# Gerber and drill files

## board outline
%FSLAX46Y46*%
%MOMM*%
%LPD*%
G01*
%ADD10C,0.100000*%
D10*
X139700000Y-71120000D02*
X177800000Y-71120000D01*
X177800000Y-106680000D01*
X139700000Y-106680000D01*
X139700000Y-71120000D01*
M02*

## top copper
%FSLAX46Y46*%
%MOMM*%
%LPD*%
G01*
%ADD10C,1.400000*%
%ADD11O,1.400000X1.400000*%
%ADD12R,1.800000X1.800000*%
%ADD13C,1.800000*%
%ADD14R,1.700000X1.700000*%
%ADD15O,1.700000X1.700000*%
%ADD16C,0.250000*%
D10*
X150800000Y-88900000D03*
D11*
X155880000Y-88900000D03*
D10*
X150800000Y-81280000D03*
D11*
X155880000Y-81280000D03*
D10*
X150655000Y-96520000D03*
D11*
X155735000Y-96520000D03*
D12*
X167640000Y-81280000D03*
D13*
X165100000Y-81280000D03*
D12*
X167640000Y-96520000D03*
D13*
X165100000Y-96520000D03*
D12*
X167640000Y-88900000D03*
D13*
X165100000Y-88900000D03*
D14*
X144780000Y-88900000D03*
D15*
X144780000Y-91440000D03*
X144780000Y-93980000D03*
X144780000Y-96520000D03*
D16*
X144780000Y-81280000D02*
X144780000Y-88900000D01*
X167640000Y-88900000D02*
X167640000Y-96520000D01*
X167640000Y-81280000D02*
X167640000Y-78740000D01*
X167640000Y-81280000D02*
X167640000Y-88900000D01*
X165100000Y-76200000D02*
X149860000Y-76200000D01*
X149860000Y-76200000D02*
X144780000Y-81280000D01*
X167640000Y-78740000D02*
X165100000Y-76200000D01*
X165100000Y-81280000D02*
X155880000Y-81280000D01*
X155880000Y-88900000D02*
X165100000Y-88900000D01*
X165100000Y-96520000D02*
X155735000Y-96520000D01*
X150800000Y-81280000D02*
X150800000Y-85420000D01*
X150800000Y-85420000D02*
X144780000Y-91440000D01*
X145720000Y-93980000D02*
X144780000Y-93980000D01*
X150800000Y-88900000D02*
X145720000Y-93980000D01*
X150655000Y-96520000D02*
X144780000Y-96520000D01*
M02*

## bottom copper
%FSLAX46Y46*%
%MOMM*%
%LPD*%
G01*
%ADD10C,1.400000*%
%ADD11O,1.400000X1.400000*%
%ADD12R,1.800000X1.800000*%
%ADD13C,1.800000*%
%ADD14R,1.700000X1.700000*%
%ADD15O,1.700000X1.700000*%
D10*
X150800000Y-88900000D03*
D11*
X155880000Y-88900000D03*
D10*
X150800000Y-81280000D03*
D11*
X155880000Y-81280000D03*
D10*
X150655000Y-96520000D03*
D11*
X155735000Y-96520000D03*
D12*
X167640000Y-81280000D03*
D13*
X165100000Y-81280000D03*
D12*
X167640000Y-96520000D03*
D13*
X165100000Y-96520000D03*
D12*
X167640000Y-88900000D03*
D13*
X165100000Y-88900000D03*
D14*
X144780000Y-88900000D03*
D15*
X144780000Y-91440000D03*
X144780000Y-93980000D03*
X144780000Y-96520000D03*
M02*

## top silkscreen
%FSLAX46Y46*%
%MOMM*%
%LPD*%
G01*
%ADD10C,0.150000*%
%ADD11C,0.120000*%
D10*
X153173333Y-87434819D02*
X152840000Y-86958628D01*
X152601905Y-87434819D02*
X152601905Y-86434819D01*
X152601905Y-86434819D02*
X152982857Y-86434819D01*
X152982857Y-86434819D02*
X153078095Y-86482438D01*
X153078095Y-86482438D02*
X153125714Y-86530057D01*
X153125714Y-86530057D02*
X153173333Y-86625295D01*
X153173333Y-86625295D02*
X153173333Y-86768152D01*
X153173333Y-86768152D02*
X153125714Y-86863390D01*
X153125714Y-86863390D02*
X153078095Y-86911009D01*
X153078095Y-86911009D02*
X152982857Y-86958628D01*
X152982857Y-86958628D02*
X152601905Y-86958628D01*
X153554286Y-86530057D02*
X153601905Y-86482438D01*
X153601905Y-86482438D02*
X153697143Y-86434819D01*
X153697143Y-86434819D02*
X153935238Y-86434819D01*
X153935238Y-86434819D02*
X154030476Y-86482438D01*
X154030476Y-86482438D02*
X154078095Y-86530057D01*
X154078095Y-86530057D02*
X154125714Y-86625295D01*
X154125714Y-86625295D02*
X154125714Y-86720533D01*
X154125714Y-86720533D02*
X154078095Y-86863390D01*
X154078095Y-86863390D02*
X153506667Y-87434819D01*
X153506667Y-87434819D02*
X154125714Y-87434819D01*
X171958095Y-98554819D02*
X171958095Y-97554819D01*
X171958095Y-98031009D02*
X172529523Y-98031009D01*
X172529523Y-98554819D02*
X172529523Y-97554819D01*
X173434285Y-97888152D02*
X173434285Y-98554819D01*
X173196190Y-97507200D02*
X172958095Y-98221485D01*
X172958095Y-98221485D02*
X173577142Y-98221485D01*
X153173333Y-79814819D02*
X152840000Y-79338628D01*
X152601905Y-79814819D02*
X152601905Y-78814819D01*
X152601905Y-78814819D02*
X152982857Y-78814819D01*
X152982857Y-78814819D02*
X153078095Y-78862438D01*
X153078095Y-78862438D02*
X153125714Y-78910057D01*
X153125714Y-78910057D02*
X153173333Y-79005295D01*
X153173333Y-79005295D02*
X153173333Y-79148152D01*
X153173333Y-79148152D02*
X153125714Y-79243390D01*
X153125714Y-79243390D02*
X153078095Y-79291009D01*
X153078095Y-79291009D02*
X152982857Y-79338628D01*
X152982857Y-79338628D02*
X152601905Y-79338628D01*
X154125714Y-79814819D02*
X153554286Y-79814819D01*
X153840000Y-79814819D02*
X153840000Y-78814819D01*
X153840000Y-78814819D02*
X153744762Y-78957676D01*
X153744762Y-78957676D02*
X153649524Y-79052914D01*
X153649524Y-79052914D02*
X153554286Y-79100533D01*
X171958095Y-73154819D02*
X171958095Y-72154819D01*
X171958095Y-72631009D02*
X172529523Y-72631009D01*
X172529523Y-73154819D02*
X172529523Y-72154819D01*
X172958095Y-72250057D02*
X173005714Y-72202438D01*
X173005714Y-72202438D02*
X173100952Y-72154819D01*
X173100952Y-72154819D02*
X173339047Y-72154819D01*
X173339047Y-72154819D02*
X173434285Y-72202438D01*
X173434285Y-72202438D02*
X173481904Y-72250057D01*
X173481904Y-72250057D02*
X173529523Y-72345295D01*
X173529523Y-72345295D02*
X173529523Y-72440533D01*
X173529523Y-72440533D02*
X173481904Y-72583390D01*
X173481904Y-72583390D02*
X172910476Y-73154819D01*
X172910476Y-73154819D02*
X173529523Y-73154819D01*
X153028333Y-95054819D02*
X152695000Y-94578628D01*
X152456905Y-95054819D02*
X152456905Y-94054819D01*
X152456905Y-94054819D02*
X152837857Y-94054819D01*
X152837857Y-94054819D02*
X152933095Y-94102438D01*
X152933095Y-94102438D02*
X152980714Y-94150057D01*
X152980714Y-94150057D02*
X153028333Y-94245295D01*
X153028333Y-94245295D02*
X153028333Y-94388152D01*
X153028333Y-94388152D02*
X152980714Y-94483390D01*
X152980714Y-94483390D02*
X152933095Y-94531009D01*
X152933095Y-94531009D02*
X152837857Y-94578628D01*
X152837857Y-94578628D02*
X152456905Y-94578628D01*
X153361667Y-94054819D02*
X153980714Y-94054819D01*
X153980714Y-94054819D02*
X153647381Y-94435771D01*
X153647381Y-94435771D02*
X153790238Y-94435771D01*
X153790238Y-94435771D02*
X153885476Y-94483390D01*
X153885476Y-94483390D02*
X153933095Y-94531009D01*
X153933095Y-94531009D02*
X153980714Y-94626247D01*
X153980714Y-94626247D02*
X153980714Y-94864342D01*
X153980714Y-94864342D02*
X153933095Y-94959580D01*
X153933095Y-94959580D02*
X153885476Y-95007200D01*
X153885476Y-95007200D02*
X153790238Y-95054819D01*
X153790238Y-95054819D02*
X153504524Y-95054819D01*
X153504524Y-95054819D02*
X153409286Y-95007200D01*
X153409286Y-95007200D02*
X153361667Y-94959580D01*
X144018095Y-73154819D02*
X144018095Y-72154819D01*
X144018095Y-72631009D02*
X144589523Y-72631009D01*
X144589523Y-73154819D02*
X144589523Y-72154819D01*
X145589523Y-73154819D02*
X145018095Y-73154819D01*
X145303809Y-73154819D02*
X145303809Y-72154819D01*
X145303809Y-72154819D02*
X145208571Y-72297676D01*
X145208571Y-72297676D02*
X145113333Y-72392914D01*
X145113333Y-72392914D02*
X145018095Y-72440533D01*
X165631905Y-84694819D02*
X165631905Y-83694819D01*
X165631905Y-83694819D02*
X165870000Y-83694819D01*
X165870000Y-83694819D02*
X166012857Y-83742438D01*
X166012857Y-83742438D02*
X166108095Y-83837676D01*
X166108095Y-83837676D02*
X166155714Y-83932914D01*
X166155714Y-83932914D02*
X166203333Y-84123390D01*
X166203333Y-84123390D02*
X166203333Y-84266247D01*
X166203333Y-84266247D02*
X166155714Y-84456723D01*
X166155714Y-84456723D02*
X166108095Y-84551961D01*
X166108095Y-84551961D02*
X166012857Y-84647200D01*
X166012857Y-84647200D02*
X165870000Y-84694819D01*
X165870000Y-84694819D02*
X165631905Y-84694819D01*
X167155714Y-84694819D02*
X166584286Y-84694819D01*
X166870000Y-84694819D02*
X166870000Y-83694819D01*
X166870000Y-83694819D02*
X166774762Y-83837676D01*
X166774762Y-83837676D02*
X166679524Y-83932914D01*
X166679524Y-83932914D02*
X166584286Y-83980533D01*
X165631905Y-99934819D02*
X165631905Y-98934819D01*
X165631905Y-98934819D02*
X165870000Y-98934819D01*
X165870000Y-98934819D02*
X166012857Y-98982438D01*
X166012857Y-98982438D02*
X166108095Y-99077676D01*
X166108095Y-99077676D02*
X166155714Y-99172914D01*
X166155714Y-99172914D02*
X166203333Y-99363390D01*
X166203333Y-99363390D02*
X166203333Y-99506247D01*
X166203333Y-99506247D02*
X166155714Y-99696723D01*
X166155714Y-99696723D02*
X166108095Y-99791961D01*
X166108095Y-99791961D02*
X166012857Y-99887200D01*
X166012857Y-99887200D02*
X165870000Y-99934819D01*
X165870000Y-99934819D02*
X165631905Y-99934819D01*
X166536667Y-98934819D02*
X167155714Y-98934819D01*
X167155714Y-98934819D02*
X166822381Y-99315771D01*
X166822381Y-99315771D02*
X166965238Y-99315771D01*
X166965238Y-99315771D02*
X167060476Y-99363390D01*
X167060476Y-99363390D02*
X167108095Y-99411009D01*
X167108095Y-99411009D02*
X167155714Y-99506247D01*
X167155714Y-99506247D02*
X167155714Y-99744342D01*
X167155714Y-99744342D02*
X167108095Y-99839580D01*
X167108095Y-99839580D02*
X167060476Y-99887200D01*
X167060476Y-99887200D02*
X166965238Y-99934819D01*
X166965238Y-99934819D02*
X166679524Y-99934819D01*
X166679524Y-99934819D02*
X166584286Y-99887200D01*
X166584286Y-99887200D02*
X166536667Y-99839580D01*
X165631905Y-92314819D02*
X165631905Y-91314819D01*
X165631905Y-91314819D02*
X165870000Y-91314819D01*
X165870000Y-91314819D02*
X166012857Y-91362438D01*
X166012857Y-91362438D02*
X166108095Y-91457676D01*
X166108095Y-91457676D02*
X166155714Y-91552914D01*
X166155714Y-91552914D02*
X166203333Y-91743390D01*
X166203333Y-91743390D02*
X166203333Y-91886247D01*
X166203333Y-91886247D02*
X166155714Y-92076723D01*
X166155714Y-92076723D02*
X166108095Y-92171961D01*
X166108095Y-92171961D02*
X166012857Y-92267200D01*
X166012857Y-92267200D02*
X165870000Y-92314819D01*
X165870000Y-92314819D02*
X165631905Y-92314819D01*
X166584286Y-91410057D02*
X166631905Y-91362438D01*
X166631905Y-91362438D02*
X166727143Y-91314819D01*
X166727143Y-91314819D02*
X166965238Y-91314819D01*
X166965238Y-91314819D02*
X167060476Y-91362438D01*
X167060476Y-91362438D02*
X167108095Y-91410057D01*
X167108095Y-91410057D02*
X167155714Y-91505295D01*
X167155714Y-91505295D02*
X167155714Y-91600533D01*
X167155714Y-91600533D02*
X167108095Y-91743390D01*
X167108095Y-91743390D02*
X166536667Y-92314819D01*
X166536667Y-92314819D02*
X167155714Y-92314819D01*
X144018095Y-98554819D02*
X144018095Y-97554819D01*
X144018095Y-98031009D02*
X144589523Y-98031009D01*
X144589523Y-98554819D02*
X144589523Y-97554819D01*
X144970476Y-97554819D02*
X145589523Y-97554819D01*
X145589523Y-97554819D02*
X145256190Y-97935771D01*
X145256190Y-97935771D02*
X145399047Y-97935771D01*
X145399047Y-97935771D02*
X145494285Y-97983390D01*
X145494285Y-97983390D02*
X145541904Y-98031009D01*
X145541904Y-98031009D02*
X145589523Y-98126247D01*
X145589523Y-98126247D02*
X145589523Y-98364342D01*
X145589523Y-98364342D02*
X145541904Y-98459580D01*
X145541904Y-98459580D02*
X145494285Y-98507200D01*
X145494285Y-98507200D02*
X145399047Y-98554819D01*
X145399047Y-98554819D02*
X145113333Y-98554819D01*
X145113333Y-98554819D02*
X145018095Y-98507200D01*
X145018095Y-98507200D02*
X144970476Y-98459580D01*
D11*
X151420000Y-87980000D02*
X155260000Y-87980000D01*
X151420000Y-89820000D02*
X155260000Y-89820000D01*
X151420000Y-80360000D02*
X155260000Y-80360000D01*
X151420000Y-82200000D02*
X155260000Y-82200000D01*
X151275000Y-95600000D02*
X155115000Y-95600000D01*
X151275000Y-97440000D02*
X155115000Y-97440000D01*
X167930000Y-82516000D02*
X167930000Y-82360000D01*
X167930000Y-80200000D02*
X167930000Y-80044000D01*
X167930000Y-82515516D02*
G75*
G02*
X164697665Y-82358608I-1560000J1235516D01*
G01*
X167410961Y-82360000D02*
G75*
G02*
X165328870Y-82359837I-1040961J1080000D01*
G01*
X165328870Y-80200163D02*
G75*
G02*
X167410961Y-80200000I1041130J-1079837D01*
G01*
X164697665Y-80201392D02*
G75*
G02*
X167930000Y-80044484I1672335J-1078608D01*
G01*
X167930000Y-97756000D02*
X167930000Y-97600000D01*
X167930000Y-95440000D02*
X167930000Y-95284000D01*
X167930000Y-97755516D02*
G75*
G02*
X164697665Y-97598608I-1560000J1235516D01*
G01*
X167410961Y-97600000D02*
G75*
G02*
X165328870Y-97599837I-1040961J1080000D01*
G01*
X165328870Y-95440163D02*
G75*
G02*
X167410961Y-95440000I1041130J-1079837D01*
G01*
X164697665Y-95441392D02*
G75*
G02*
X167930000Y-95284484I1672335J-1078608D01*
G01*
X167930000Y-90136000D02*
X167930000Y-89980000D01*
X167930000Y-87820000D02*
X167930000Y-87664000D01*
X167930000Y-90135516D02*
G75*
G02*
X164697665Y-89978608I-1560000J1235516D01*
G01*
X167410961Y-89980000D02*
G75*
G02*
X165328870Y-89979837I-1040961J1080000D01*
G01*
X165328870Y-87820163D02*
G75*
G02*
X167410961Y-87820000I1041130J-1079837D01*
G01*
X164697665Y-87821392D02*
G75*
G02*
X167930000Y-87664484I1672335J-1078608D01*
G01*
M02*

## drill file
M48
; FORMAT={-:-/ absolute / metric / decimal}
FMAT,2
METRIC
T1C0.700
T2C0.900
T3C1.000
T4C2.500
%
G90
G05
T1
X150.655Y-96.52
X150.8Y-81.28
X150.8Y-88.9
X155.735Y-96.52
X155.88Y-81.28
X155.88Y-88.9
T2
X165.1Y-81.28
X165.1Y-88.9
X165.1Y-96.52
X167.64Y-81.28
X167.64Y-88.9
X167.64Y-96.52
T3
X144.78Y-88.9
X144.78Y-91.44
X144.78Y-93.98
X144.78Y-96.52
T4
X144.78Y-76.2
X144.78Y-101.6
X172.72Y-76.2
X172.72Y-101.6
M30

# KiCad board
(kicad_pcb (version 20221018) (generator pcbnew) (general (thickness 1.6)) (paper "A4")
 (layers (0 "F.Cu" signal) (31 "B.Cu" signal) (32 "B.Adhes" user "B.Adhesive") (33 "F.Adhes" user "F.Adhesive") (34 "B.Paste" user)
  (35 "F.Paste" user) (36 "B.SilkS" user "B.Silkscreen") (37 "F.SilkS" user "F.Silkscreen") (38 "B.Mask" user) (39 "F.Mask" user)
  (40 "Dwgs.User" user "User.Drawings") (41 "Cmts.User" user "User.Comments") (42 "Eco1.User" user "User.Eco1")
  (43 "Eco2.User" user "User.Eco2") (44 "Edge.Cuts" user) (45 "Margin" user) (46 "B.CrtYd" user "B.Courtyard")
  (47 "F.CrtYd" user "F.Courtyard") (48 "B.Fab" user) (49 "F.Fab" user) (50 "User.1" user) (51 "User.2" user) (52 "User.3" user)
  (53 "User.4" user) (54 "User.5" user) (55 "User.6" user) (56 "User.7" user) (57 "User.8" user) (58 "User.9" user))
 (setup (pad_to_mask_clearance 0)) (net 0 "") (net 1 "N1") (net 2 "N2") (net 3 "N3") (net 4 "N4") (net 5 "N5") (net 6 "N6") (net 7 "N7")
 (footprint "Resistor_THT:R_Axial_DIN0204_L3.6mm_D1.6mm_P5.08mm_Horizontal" (layer "F.Cu") (at 150.8 88.9)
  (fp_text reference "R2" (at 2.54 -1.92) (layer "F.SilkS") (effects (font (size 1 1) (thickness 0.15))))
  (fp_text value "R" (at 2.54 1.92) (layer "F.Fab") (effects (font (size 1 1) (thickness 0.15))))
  (fp_line (start 0.62 -0.92) (end 4.46 -0.92) (stroke (width 0.12) (type solid)) (layer "F.SilkS"))
  (fp_line (start 0.62 0.92) (end 4.46 0.92) (stroke (width 0.12) (type solid)) (layer "F.SilkS"))
  (pad "1" thru_hole circle (at 0 0) (size 1.4 1.4) (drill 0.7) (layers "*.Cu" "*.Mask") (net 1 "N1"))
  (pad "2" thru_hole oval (at 5.08 0) (size 1.4 1.4) (drill 0.7) (layers "*.Cu" "*.Mask") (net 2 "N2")))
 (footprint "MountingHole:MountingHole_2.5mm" (layer "F.Cu") (at 172.72 101.6)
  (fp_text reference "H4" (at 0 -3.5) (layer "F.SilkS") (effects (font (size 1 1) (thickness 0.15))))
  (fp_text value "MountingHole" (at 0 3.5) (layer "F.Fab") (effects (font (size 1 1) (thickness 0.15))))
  (pad "" np_thru_hole circle (at 0 0) (size 2.5 2.5) (drill 2.5) (layers "*.Cu" "*.Mask")))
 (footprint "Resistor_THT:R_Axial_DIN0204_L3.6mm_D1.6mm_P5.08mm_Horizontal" (layer "F.Cu") (at 150.8 81.28)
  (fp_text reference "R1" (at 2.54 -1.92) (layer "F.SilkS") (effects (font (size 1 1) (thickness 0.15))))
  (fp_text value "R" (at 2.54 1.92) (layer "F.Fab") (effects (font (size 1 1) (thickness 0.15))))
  (fp_line (start 0.62 -0.92) (end 4.46 -0.92) (stroke (width 0.12) (type solid)) (layer "F.SilkS"))
  (fp_line (start 0.62 0.92) (end 4.46 0.92) (stroke (width 0.12) (type solid)) (layer "F.SilkS"))
  (pad "1" thru_hole circle (at 0 0) (size 1.4 1.4) (drill 0.7) (layers "*.Cu" "*.Mask") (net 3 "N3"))
  (pad "2" thru_hole oval (at 5.08 0) (size 1.4 1.4) (drill 0.7) (layers "*.Cu" "*.Mask") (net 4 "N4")))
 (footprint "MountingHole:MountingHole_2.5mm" (layer "F.Cu") (at 172.72 76.2)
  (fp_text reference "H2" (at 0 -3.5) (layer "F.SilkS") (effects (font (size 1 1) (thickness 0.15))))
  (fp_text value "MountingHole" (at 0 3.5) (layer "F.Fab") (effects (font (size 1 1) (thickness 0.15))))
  (pad "" np_thru_hole circle (at 0 0) (size 2.5 2.5) (drill 2.5) (layers "*.Cu" "*.Mask")))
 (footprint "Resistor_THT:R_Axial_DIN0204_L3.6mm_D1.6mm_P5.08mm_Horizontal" (layer "F.Cu") (at 150.655 96.52)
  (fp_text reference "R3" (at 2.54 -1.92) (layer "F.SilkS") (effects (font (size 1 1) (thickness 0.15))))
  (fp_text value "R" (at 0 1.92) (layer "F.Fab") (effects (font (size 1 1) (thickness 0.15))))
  (fp_line (start 0.62 -0.92) (end 4.46 -0.92) (stroke (width 0.12) (type solid)) (layer "F.SilkS"))
  (fp_line (start 0.62 0.92) (end 4.46 0.92) (stroke (width 0.12) (type solid)) (layer "F.SilkS"))
  (pad "1" thru_hole circle (at 0 0) (size 1.4 1.4) (drill 0.7) (layers "*.Cu" "*.Mask") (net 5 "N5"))
  (pad "2" thru_hole oval (at 5.08 0) (size 1.4 1.4) (drill 0.7) (layers "*.Cu" "*.Mask") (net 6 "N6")))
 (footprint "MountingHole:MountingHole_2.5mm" (layer "F.Cu") (at 144.78 76.2)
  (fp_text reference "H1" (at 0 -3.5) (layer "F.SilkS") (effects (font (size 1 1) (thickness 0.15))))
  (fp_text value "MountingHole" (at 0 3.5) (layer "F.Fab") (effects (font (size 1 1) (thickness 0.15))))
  (pad "" np_thru_hole circle (at 0 0) (size 2.5 2.5) (drill 2.5) (layers "*.Cu" "*.Mask")))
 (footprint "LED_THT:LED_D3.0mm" (layer "F.Cu") (at 167.64 81.28 180)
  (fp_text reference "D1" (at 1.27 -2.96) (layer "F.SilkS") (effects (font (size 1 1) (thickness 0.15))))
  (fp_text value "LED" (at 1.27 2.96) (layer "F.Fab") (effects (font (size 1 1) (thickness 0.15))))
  (fp_line (start -0.29 -1.236) (end -0.29 -1.08) (stroke (width 0.12) (type solid)) (layer "F.SilkS"))
  (fp_line (start -0.29 1.08) (end -0.29 1.236) (stroke (width 0.12) (type solid)) (layer "F.SilkS"))
  (fp_arc (start -0.29 -1.235516) (mid 1.366487 -1.987659) (end 2.942335 -1.078608) (stroke (width 0.12) (type solid)) (layer "F.SilkS"))
  (fp_arc (start 0.229039 -1.08) (mid 1.270117 -1.5) (end 2.31113 -1.079837) (stroke (width 0.12) (type solid)) (layer "F.SilkS"))
  (fp_arc (start 2.31113 1.079837) (mid 1.270117 1.5) (end 0.229039 1.08) (stroke (width 0.12) (type solid)) (layer "F.SilkS"))
  (fp_arc (start 2.942335 1.078608) (mid 1.366487 1.987659) (end -0.29 1.235516) (stroke (width 0.12) (type solid)) (layer "F.SilkS"))
  (pad "1" thru_hole rect (at 0 0 180) (size 1.8 1.8) (drill 0.9) (layers "*.Cu" "*.Mask") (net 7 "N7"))
  (pad "2" thru_hole circle (at 2.54 0 180) (size 1.8 1.8) (drill 0.9) (layers "*.Cu" "*.Mask") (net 4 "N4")))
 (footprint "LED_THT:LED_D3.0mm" (layer "F.Cu") (at 167.64 96.52 180)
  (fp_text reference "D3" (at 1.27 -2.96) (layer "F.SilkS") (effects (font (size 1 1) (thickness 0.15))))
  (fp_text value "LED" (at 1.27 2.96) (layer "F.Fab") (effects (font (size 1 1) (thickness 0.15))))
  (fp_line (start -0.29 -1.236) (end -0.29 -1.08) (stroke (width 0.12) (type solid)) (layer "F.SilkS"))
  (fp_line (start -0.29 1.08) (end -0.29 1.236) (stroke (width 0.12) (type solid)) (layer "F.SilkS"))
  (fp_arc (start -0.29 -1.235516) (mid 1.366487 -1.987659) (end 2.942335 -1.078608) (stroke (width 0.12) (type solid)) (layer "F.SilkS"))
  (fp_arc (start 0.229039 -1.08) (mid 1.270117 -1.5) (end 2.31113 -1.079837) (stroke (width 0.12) (type solid)) (layer "F.SilkS"))
  (fp_arc (start 2.31113 1.079837) (mid 1.270117 1.5) (end 0.229039 1.08) (stroke (width 0.12) (type solid)) (layer "F.SilkS"))
  (fp_arc (start 2.942335 1.078608) (mid 1.366487 1.987659) (end -0.29 1.235516) (stroke (width 0.12) (type solid)) (layer "F.SilkS"))
  (pad "1" thru_hole rect (at 0 0 180) (size 1.8 1.8) (drill 0.9) (layers "*.Cu" "*.Mask") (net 7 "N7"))
  (pad "2" thru_hole circle (at 2.54 0 180) (size 1.8 1.8) (drill 0.9) (layers "*.Cu" "*.Mask") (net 6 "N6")))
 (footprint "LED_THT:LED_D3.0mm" (layer "F.Cu") (at 167.64 88.9 180)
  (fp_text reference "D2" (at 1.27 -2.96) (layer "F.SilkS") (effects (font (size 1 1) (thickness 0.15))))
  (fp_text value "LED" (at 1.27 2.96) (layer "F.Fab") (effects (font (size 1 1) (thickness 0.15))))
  (fp_line (start -0.29 -1.236) (end -0.29 -1.08) (stroke (width 0.12) (type solid)) (layer "F.SilkS"))
  (fp_line (start -0.29 1.08) (end -0.29 1.236) (stroke (width 0.12) (type solid)) (layer "F.SilkS"))
  (fp_arc (start -0.29 -1.235516) (mid 1.366487 -1.987659) (end 2.942335 -1.078608) (stroke (width 0.12) (type solid)) (layer "F.SilkS"))
  (fp_arc (start 0.229039 -1.08) (mid 1.270117 -1.5) (end 2.31113 -1.079837) (stroke (width 0.12) (type solid)) (layer "F.SilkS"))
  (fp_arc (start 2.31113 1.079837) (mid 1.270117 1.5) (end 0.229039 1.08) (stroke (width 0.12) (type solid)) (layer "F.SilkS"))
  (fp_arc (start 2.942335 1.078608) (mid 1.366487 1.987659) (end -0.29 1.235516) (stroke (width 0.12) (type solid)) (layer "F.SilkS"))
  (pad "1" thru_hole rect (at 0 0 180) (size 1.8 1.8) (drill 0.9) (layers "*.Cu" "*.Mask") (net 7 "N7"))
  (pad "2" thru_hole circle (at 2.54 0 180) (size 1.8 1.8) (drill 0.9) (layers "*.Cu" "*.Mask") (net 2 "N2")))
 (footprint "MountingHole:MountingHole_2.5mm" (layer "F.Cu") (at 144.78 101.6)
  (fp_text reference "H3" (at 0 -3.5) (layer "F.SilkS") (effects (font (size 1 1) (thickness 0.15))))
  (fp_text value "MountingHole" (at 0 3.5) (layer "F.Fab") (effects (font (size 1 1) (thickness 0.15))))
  (pad "" np_thru_hole circle (at 0 0) (size 2.5 2.5) (drill 2.5) (layers "*.Cu" "*.Mask")))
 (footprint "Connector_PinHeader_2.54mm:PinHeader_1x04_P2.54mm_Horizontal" (layer "B.Cu") (at 144.78 88.9 180)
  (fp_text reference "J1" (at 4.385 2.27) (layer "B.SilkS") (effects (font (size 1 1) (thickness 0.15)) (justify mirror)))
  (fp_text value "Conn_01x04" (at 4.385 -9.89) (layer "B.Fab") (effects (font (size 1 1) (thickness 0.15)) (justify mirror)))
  (pad "1" thru_hole rect (at 0 0 180) (size 1.7 1.7) (drill 1) (layers "*.Cu" "*.Mask") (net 7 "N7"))
  (pad "2" thru_hole oval (at 0 -2.54 180) (size 1.7 1.7) (drill 1) (layers "*.Cu" "*.Mask") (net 3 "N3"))
  (pad "3" thru_hole oval (at 0 -5.08 180) (size 1.7 1.7) (drill 1) (layers "*.Cu" "*.Mask") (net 1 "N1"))
  (pad "4" thru_hole oval (at 0 -7.62 180) (size 1.7 1.7) (drill 1) (layers "*.Cu" "*.Mask") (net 5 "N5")))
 (gr_poly
  (pts (xy 139.7 71.12) (xy 177.8 71.12) (xy 177.8 106.68) (xy 139.7 106.68)) (stroke (width 0.1) (type solid)) (fill none)
  (layer "Edge.Cuts"))
 (segment (start 144.78 81.28) (end 144.78 88.9) (width 0.25) (layer "F.Cu") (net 7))
 (segment (start 167.64 88.9) (end 167.64 96.52) (width 0.25) (layer "F.Cu") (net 7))
 (segment (start 167.64 81.28) (end 167.64 78.74) (width 0.25) (layer "F.Cu") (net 7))
 (segment (start 167.64 81.28) (end 167.64 88.9) (width 0.25) (layer "F.Cu") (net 7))
 (segment (start 165.1 76.2) (end 149.86 76.2) (width 0.25) (layer "F.Cu") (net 7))
 (segment (start 149.86 76.2) (end 144.78 81.28) (width 0.25) (layer "F.Cu") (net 7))
 (segment (start 167.64 78.74) (end 165.1 76.2) (width 0.25) (layer "F.Cu") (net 7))
 (segment (start 165.1 81.28) (end 155.88 81.28) (width 0.25) (layer "F.Cu") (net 4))
 (segment (start 155.88 88.9) (end 165.1 88.9) (width 0.25) (layer "F.Cu") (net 2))
 (segment (start 165.1 96.52) (end 155.735 96.52) (width 0.25) (layer "F.Cu") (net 6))
 (segment (start 150.8 81.28) (end 150.8 85.42) (width 0.25) (layer "F.Cu") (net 3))
 (segment (start 150.8 85.42) (end 144.78 91.44) (width 0.25) (layer "F.Cu") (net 3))
 (segment (start 145.72 93.98) (end 144.78 93.98) (width 0.25) (layer "F.Cu") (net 1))
 (segment (start 150.8 88.9) (end 145.72 93.98) (width 0.25) (layer "F.Cu") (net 1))
 (segment (start 150.655 96.52) (end 144.78 96.52) (width 0.25) (layer "F.Cu") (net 5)))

